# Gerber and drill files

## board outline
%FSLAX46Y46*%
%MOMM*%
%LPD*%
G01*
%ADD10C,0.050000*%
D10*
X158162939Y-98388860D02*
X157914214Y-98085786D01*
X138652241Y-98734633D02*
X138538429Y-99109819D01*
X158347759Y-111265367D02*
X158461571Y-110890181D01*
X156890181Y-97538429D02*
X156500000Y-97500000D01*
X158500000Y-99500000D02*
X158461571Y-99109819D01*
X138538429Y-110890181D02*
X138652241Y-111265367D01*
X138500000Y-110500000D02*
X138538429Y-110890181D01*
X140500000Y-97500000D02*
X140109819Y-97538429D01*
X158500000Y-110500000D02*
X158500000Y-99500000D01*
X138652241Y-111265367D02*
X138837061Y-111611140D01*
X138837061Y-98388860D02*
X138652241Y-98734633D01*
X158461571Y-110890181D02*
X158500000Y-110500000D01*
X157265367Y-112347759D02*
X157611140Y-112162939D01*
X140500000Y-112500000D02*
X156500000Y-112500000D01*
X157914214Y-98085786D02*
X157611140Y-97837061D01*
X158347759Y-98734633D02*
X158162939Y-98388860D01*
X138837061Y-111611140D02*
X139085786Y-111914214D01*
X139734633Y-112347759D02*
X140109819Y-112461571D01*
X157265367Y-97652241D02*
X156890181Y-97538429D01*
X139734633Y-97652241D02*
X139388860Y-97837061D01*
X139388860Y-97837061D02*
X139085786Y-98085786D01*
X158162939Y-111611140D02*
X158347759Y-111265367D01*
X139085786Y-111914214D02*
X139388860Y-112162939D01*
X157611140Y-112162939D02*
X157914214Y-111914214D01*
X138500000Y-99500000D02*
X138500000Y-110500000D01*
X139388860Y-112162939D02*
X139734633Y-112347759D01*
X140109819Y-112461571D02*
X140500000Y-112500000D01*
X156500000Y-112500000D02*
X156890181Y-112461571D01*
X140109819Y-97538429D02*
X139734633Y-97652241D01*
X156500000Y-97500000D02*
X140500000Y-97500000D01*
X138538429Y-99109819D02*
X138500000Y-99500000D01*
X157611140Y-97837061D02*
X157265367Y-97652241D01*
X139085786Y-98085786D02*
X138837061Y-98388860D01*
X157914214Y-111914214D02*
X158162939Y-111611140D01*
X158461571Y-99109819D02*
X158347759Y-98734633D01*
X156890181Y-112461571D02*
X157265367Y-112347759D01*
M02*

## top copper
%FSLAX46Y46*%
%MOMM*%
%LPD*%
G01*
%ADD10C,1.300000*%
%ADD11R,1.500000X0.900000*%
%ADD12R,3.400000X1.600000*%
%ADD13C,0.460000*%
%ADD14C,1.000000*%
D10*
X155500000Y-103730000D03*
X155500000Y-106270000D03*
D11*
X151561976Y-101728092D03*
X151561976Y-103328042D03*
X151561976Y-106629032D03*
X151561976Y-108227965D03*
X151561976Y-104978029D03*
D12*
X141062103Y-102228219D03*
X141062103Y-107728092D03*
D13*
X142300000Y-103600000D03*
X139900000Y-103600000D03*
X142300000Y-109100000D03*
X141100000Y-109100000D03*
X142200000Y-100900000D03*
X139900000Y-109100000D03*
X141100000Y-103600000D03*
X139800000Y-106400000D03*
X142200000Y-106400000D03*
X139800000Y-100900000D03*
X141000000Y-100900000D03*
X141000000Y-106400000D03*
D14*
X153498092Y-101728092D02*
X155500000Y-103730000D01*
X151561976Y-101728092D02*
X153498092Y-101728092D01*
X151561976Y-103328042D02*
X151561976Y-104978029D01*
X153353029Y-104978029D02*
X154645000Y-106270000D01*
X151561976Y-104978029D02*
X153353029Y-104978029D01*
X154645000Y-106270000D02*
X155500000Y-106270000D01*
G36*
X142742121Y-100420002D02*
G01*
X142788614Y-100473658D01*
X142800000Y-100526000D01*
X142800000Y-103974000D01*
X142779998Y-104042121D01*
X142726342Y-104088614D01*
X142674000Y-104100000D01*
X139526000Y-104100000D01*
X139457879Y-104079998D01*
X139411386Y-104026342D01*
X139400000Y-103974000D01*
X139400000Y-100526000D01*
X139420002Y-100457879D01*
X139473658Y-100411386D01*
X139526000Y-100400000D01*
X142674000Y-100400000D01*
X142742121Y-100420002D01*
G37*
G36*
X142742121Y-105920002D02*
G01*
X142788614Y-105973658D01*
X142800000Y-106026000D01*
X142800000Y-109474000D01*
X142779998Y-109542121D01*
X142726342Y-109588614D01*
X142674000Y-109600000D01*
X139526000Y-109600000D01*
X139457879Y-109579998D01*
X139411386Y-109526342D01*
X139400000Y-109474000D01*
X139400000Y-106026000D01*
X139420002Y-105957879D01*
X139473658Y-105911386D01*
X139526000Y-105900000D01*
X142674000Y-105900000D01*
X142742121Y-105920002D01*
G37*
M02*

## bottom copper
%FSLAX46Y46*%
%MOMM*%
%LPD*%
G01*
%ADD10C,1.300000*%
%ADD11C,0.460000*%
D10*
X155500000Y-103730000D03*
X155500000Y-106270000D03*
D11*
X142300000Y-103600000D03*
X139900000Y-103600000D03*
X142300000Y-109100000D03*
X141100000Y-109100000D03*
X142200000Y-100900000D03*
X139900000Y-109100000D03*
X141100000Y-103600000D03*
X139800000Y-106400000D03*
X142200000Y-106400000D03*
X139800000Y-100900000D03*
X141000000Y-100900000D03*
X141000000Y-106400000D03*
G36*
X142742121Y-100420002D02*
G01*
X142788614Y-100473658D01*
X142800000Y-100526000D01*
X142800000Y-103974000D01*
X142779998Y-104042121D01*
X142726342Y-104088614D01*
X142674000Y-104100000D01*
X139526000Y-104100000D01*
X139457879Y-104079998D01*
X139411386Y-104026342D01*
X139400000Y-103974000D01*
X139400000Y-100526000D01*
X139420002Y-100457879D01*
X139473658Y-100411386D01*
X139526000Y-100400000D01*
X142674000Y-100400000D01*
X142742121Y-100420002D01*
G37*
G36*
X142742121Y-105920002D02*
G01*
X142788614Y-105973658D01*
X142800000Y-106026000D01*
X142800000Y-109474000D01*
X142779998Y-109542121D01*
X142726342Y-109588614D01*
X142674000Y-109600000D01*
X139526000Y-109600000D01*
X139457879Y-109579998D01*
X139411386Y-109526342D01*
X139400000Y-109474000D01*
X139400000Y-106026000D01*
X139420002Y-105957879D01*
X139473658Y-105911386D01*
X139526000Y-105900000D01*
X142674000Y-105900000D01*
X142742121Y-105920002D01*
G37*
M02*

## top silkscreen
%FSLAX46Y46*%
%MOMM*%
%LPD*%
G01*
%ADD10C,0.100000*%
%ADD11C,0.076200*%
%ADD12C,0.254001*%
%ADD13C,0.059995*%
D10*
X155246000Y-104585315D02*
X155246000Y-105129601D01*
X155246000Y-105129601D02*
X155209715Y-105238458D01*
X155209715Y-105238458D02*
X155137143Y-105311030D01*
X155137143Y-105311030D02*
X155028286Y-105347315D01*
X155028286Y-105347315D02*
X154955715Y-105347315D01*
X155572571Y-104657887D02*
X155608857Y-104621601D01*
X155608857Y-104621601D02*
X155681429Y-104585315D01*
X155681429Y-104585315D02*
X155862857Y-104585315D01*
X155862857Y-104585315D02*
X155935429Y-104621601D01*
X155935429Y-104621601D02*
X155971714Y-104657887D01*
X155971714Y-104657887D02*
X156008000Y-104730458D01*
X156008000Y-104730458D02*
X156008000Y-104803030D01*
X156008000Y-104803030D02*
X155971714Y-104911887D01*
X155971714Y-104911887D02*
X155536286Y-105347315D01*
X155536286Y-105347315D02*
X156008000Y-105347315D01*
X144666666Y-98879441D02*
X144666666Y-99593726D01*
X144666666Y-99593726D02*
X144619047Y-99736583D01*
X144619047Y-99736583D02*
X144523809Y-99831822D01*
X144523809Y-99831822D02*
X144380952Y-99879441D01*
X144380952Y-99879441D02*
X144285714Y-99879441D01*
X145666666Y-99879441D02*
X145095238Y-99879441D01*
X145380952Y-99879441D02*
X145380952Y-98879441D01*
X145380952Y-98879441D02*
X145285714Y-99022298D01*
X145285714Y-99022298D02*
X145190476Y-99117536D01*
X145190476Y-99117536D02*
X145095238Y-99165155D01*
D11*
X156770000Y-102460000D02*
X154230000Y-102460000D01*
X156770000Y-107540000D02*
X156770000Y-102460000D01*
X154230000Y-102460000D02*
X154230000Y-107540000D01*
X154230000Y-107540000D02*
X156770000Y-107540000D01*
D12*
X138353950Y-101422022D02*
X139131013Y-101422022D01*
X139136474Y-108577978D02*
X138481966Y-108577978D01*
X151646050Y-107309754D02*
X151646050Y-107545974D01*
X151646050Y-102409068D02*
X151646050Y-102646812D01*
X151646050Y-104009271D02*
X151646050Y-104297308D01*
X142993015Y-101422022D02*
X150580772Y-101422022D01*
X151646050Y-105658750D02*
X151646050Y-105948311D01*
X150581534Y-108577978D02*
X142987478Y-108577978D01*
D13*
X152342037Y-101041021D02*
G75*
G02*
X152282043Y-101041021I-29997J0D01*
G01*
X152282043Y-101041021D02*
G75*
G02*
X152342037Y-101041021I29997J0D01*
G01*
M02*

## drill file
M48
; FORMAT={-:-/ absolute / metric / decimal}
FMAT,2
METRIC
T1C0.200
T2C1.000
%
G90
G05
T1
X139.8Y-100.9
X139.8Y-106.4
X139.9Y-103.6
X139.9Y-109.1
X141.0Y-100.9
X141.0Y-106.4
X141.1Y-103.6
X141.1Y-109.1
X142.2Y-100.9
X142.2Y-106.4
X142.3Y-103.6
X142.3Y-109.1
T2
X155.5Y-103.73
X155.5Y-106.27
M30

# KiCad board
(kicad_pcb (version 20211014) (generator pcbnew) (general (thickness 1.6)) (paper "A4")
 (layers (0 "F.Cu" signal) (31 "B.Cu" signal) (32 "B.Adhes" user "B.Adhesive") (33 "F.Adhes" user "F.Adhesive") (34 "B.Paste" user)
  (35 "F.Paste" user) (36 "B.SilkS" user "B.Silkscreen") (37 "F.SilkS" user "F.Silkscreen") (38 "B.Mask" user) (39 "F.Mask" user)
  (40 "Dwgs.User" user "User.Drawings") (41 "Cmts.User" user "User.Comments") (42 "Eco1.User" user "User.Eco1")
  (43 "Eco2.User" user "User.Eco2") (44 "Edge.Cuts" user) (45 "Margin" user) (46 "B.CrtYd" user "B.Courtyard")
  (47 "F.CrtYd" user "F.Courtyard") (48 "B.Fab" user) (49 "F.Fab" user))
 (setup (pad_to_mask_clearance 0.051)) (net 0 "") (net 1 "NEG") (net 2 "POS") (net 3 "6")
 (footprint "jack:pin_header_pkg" (layer "F.Cu") (at 155.5 105)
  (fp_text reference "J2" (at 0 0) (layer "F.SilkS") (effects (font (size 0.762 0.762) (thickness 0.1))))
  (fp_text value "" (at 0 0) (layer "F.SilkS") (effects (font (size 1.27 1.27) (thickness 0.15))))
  (fp_line (start 1.27 -2.54) (end -1.27 -2.54) (layer "F.SilkS") (width 0.0762))
  (fp_line (start 1.27 2.54) (end 1.27 -2.54) (layer "F.SilkS") (width 0.0762))
  (fp_line (start -1.27 -2.54) (end -1.27 2.54) (layer "F.SilkS") (width 0.0762))
  (fp_line (start -1.27 2.54) (end 1.27 2.54) (layer "F.SilkS") (width 0.0762))
  (pad "1" thru_hole circle locked (at 0 -1.27) (size 1.3 1.3) (drill 1) (layers *.Cu) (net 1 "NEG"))
  (pad "2" thru_hole circle locked (at 0 1.27) (size 1.3 1.3) (drill 1) (layers *.Cu) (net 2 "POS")))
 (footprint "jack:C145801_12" (layer "F.Cu") (at 145 105)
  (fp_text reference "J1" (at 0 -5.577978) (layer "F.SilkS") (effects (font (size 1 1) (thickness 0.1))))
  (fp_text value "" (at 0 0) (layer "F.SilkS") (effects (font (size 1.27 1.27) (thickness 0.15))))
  (fp_line (start -6.64605 -3.577978) (end -5.868987 -3.577978) (layer "F.SilkS") (width 0.254001))
  (fp_line (start -5.863526 3.577978) (end -6.518034 3.577978) (layer "F.SilkS") (width 0.254001))
  (fp_line (start 6.64605 2.309754) (end 6.64605 2.545974) (layer "F.SilkS") (width 0.254001))
  (fp_line (start 6.64605 -2.590932) (end 6.64605 -2.353188) (layer "F.SilkS") (width 0.254001))
  (fp_line (start 6.64605 -0.990729) (end 6.64605 -0.702692) (layer "F.SilkS") (width 0.254001))
  (fp_line (start -2.006985 -3.577978) (end 5.580772 -3.577978) (layer "F.SilkS") (width 0.254001))
  (fp_line (start 6.64605 0.65875) (end 6.64605 0.948311) (layer "F.SilkS") (width 0.254001))
  (fp_line (start 5.581534 3.577978) (end -2.012522 3.577978) (layer "F.SilkS") (width 0.254001))
  (fp_arc (start 7.342037 -3.958979) (mid 7.282043 -3.958979) (end 7.342037 -3.958979) (layer "F.SilkS") (width 0.059995))
  (pad "1" smd rect locked (at 6.561976 -3.271908) (size 1.5 0.9) (layers "F.Cu" "F.Paste" "F.Mask") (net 1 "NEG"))
  (pad "2" smd rect locked (at 6.561976 -1.671958) (size 1.5 0.9) (layers "F.Cu" "F.Paste" "F.Mask") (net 2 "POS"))
  (pad "3" smd rect locked (at 6.561976 1.629032) (size 1.5 0.9) (layers "F.Cu" "F.Paste" "F.Mask"))
  (pad "4" smd rect locked (at 6.561976 3.227965) (size 1.5 0.9) (layers "F.Cu" "F.Paste" "F.Mask"))
  (pad "5" smd rect locked (at 6.561976 -0.021971) (size 1.5 0.9) (layers "F.Cu" "F.Paste" "F.Mask") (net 2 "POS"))
  (pad "6" smd rect locked (at -3.937897 -2.771781) (size 3.4 1.6) (layers "F.Cu" "F.Paste" "F.Mask") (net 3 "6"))
  (pad "7" smd rect locked (at -3.937897 2.728092) (size 3.4 1.6) (layers "F.Cu" "F.Paste" "F.Mask") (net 3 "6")))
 (gr_line (start 158.162939 98.38886) (end 157.914214 98.085786) (layer "Edge.Cuts") (width 0.05))
 (gr_line (start 138.652241 98.734633) (end 138.538429 99.109819) (layer "Edge.Cuts") (width 0.05))
 (gr_line (start 158.347759 111.265367) (end 158.461571 110.890181) (layer "Edge.Cuts") (width 0.05))
 (gr_line (start 156.890181 97.538429) (end 156.5 97.5) (layer "Edge.Cuts") (width 0.05))
 (gr_line (start 158.5 99.5) (end 158.461571 99.109819) (layer "Edge.Cuts") (width 0.05))
 (gr_line (start 138.538429 110.890181) (end 138.652241 111.265367) (layer "Edge.Cuts") (width 0.05))
 (gr_line (start 138.5 110.5) (end 138.538429 110.890181) (layer "Edge.Cuts") (width 0.05))
 (gr_line (start 140.5 97.5) (end 140.109819 97.538429) (layer "Edge.Cuts") (width 0.05))
 (gr_line (start 158.5 110.5) (end 158.5 99.5) (layer "Edge.Cuts") (width 0.05))
 (gr_line (start 138.652241 111.265367) (end 138.837061 111.61114) (layer "Edge.Cuts") (width 0.05))
 (gr_line (start 138.837061 98.38886) (end 138.652241 98.734633) (layer "Edge.Cuts") (width 0.05))
 (gr_line (start 158.461571 110.890181) (end 158.5 110.5) (layer "Edge.Cuts") (width 0.05))
 (gr_line (start 157.265367 112.347759) (end 157.61114 112.162939) (layer "Edge.Cuts") (width 0.05))
 (gr_line (start 140.5 112.5) (end 156.5 112.5) (layer "Edge.Cuts") (width 0.05))
 (gr_line (start 157.914214 98.085786) (end 157.61114 97.837061) (layer "Edge.Cuts") (width 0.05))
 (gr_line (start 158.347759 98.734633) (end 158.162939 98.38886) (layer "Edge.Cuts") (width 0.05))
 (gr_line (start 138.837061 111.61114) (end 139.085786 111.914214) (layer "Edge.Cuts") (width 0.05))
 (gr_line (start 139.734633 112.347759) (end 140.109819 112.461571) (layer "Edge.Cuts") (width 0.05))
 (gr_line (start 157.265367 97.652241) (end 156.890181 97.538429) (layer "Edge.Cuts") (width 0.05))
 (gr_line (start 139.734633 97.652241) (end 139.38886 97.837061) (layer "Edge.Cuts") (width 0.05))
 (gr_line (start 139.38886 97.837061) (end 139.085786 98.085786) (layer "Edge.Cuts") (width 0.05))
 (gr_line (start 158.162939 111.61114) (end 158.347759 111.265367) (layer "Edge.Cuts") (width 0.05))
 (gr_line (start 139.085786 111.914214) (end 139.38886 112.162939) (layer "Edge.Cuts") (width 0.05))
 (gr_line (start 157.61114 112.162939) (end 157.914214 111.914214) (layer "Edge.Cuts") (width 0.05))
 (gr_line (start 138.5 99.5) (end 138.5 110.5) (layer "Edge.Cuts") (width 0.05))
 (gr_line (start 139.38886 112.162939) (end 139.734633 112.347759) (layer "Edge.Cuts") (width 0.05))
 (gr_line (start 140.109819 112.461571) (end 140.5 112.5) (layer "Edge.Cuts") (width 0.05))
 (gr_line (start 156.5 112.5) (end 156.890181 112.461571) (layer "Edge.Cuts") (width 0.05))
 (gr_line (start 140.109819 97.538429) (end 139.734633 97.652241) (layer "Edge.Cuts") (width 0.05))
 (gr_line (start 156.5 97.5) (end 140.5 97.5) (layer "Edge.Cuts") (width 0.05))
 (gr_line (start 138.538429 99.109819) (end 138.5 99.5) (layer "Edge.Cuts") (width 0.05))
 (gr_line (start 157.61114 97.837061) (end 157.265367 97.652241) (layer "Edge.Cuts") (width 0.05))
 (gr_line (start 139.085786 98.085786) (end 138.837061 98.38886) (layer "Edge.Cuts") (width 0.05))
 (gr_line (start 157.914214 111.914214) (end 158.162939 111.61114) (layer "Edge.Cuts") (width 0.05))
 (gr_line (start 158.461571 99.109819) (end 158.347759 98.734633) (layer "Edge.Cuts") (width 0.05))
 (gr_line (start 156.890181 112.461571) (end 157.265367 112.347759) (layer "Edge.Cuts") (width 0.05))
 (segment (start 153.498092 101.728092) (end 155.5 103.73) (width 1) (layer "F.Cu") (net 1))
 (segment (start 151.561976 101.728092) (end 153.498092 101.728092) (width 1) (layer "F.Cu") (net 1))
 (segment (start 151.561976 103.328042) (end 151.561976 104.978029) (width 1) (layer "F.Cu") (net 2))
 (segment (start 153.353029 104.978029) (end 154.645 106.27) (width 1) (layer "F.Cu") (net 2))
 (segment (start 151.561976 104.978029) (end 153.353029 104.978029) (width 1) (layer "F.Cu") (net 2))
 (segment (start 154.645 106.27) (end 155.5 106.27) (width 1) (layer "F.Cu") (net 2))
 (via (at 142.3 103.6) (size 0.46) (drill 0.2) (layers "F.Cu" "B.Cu") (free) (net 3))
 (via (at 139.9 103.6) (size 0.46) (drill 0.2) (layers "F.Cu" "B.Cu") (free) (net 3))
 (via (at 142.3 109.1) (size 0.46) (drill 0.2) (layers "F.Cu" "B.Cu") (free) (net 3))
 (via (at 141.1 109.1) (size 0.46) (drill 0.2) (layers "F.Cu" "B.Cu") (free) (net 3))
 (via (at 142.2 100.9) (size 0.46) (drill 0.2) (layers "F.Cu" "B.Cu") (free) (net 3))
 (via (at 139.9 109.1) (size 0.46) (drill 0.2) (layers "F.Cu" "B.Cu") (free) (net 3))
 (via (at 141.1 103.6) (size 0.46) (drill 0.2) (layers "F.Cu" "B.Cu") (free) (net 3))
 (via (at 139.8 106.4) (size 0.46) (drill 0.2) (layers "F.Cu" "B.Cu") (free) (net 3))
 (via (at 142.2 106.4) (size 0.46) (drill 0.2) (layers "F.Cu" "B.Cu") (free) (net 3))
 (via (at 139.8 100.9) (size 0.46) (drill 0.2) (layers "F.Cu" "B.Cu") (free) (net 3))
 (via (at 141 100.9) (size 0.46) (drill 0.2) (layers "F.Cu" "B.Cu") (free) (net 3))
 (via (at 141 106.4) (size 0.46) (drill 0.2) (layers "F.Cu" "B.Cu") (free) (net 3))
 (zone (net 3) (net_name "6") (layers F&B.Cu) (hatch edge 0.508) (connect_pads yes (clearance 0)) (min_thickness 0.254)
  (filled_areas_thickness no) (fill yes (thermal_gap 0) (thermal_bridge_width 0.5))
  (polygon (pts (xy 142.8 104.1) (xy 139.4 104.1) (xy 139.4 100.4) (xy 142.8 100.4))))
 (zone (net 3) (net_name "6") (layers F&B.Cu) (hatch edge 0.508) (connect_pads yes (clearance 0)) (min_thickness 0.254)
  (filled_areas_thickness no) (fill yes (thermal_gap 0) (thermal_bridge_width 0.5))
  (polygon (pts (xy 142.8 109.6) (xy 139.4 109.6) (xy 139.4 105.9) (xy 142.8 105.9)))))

